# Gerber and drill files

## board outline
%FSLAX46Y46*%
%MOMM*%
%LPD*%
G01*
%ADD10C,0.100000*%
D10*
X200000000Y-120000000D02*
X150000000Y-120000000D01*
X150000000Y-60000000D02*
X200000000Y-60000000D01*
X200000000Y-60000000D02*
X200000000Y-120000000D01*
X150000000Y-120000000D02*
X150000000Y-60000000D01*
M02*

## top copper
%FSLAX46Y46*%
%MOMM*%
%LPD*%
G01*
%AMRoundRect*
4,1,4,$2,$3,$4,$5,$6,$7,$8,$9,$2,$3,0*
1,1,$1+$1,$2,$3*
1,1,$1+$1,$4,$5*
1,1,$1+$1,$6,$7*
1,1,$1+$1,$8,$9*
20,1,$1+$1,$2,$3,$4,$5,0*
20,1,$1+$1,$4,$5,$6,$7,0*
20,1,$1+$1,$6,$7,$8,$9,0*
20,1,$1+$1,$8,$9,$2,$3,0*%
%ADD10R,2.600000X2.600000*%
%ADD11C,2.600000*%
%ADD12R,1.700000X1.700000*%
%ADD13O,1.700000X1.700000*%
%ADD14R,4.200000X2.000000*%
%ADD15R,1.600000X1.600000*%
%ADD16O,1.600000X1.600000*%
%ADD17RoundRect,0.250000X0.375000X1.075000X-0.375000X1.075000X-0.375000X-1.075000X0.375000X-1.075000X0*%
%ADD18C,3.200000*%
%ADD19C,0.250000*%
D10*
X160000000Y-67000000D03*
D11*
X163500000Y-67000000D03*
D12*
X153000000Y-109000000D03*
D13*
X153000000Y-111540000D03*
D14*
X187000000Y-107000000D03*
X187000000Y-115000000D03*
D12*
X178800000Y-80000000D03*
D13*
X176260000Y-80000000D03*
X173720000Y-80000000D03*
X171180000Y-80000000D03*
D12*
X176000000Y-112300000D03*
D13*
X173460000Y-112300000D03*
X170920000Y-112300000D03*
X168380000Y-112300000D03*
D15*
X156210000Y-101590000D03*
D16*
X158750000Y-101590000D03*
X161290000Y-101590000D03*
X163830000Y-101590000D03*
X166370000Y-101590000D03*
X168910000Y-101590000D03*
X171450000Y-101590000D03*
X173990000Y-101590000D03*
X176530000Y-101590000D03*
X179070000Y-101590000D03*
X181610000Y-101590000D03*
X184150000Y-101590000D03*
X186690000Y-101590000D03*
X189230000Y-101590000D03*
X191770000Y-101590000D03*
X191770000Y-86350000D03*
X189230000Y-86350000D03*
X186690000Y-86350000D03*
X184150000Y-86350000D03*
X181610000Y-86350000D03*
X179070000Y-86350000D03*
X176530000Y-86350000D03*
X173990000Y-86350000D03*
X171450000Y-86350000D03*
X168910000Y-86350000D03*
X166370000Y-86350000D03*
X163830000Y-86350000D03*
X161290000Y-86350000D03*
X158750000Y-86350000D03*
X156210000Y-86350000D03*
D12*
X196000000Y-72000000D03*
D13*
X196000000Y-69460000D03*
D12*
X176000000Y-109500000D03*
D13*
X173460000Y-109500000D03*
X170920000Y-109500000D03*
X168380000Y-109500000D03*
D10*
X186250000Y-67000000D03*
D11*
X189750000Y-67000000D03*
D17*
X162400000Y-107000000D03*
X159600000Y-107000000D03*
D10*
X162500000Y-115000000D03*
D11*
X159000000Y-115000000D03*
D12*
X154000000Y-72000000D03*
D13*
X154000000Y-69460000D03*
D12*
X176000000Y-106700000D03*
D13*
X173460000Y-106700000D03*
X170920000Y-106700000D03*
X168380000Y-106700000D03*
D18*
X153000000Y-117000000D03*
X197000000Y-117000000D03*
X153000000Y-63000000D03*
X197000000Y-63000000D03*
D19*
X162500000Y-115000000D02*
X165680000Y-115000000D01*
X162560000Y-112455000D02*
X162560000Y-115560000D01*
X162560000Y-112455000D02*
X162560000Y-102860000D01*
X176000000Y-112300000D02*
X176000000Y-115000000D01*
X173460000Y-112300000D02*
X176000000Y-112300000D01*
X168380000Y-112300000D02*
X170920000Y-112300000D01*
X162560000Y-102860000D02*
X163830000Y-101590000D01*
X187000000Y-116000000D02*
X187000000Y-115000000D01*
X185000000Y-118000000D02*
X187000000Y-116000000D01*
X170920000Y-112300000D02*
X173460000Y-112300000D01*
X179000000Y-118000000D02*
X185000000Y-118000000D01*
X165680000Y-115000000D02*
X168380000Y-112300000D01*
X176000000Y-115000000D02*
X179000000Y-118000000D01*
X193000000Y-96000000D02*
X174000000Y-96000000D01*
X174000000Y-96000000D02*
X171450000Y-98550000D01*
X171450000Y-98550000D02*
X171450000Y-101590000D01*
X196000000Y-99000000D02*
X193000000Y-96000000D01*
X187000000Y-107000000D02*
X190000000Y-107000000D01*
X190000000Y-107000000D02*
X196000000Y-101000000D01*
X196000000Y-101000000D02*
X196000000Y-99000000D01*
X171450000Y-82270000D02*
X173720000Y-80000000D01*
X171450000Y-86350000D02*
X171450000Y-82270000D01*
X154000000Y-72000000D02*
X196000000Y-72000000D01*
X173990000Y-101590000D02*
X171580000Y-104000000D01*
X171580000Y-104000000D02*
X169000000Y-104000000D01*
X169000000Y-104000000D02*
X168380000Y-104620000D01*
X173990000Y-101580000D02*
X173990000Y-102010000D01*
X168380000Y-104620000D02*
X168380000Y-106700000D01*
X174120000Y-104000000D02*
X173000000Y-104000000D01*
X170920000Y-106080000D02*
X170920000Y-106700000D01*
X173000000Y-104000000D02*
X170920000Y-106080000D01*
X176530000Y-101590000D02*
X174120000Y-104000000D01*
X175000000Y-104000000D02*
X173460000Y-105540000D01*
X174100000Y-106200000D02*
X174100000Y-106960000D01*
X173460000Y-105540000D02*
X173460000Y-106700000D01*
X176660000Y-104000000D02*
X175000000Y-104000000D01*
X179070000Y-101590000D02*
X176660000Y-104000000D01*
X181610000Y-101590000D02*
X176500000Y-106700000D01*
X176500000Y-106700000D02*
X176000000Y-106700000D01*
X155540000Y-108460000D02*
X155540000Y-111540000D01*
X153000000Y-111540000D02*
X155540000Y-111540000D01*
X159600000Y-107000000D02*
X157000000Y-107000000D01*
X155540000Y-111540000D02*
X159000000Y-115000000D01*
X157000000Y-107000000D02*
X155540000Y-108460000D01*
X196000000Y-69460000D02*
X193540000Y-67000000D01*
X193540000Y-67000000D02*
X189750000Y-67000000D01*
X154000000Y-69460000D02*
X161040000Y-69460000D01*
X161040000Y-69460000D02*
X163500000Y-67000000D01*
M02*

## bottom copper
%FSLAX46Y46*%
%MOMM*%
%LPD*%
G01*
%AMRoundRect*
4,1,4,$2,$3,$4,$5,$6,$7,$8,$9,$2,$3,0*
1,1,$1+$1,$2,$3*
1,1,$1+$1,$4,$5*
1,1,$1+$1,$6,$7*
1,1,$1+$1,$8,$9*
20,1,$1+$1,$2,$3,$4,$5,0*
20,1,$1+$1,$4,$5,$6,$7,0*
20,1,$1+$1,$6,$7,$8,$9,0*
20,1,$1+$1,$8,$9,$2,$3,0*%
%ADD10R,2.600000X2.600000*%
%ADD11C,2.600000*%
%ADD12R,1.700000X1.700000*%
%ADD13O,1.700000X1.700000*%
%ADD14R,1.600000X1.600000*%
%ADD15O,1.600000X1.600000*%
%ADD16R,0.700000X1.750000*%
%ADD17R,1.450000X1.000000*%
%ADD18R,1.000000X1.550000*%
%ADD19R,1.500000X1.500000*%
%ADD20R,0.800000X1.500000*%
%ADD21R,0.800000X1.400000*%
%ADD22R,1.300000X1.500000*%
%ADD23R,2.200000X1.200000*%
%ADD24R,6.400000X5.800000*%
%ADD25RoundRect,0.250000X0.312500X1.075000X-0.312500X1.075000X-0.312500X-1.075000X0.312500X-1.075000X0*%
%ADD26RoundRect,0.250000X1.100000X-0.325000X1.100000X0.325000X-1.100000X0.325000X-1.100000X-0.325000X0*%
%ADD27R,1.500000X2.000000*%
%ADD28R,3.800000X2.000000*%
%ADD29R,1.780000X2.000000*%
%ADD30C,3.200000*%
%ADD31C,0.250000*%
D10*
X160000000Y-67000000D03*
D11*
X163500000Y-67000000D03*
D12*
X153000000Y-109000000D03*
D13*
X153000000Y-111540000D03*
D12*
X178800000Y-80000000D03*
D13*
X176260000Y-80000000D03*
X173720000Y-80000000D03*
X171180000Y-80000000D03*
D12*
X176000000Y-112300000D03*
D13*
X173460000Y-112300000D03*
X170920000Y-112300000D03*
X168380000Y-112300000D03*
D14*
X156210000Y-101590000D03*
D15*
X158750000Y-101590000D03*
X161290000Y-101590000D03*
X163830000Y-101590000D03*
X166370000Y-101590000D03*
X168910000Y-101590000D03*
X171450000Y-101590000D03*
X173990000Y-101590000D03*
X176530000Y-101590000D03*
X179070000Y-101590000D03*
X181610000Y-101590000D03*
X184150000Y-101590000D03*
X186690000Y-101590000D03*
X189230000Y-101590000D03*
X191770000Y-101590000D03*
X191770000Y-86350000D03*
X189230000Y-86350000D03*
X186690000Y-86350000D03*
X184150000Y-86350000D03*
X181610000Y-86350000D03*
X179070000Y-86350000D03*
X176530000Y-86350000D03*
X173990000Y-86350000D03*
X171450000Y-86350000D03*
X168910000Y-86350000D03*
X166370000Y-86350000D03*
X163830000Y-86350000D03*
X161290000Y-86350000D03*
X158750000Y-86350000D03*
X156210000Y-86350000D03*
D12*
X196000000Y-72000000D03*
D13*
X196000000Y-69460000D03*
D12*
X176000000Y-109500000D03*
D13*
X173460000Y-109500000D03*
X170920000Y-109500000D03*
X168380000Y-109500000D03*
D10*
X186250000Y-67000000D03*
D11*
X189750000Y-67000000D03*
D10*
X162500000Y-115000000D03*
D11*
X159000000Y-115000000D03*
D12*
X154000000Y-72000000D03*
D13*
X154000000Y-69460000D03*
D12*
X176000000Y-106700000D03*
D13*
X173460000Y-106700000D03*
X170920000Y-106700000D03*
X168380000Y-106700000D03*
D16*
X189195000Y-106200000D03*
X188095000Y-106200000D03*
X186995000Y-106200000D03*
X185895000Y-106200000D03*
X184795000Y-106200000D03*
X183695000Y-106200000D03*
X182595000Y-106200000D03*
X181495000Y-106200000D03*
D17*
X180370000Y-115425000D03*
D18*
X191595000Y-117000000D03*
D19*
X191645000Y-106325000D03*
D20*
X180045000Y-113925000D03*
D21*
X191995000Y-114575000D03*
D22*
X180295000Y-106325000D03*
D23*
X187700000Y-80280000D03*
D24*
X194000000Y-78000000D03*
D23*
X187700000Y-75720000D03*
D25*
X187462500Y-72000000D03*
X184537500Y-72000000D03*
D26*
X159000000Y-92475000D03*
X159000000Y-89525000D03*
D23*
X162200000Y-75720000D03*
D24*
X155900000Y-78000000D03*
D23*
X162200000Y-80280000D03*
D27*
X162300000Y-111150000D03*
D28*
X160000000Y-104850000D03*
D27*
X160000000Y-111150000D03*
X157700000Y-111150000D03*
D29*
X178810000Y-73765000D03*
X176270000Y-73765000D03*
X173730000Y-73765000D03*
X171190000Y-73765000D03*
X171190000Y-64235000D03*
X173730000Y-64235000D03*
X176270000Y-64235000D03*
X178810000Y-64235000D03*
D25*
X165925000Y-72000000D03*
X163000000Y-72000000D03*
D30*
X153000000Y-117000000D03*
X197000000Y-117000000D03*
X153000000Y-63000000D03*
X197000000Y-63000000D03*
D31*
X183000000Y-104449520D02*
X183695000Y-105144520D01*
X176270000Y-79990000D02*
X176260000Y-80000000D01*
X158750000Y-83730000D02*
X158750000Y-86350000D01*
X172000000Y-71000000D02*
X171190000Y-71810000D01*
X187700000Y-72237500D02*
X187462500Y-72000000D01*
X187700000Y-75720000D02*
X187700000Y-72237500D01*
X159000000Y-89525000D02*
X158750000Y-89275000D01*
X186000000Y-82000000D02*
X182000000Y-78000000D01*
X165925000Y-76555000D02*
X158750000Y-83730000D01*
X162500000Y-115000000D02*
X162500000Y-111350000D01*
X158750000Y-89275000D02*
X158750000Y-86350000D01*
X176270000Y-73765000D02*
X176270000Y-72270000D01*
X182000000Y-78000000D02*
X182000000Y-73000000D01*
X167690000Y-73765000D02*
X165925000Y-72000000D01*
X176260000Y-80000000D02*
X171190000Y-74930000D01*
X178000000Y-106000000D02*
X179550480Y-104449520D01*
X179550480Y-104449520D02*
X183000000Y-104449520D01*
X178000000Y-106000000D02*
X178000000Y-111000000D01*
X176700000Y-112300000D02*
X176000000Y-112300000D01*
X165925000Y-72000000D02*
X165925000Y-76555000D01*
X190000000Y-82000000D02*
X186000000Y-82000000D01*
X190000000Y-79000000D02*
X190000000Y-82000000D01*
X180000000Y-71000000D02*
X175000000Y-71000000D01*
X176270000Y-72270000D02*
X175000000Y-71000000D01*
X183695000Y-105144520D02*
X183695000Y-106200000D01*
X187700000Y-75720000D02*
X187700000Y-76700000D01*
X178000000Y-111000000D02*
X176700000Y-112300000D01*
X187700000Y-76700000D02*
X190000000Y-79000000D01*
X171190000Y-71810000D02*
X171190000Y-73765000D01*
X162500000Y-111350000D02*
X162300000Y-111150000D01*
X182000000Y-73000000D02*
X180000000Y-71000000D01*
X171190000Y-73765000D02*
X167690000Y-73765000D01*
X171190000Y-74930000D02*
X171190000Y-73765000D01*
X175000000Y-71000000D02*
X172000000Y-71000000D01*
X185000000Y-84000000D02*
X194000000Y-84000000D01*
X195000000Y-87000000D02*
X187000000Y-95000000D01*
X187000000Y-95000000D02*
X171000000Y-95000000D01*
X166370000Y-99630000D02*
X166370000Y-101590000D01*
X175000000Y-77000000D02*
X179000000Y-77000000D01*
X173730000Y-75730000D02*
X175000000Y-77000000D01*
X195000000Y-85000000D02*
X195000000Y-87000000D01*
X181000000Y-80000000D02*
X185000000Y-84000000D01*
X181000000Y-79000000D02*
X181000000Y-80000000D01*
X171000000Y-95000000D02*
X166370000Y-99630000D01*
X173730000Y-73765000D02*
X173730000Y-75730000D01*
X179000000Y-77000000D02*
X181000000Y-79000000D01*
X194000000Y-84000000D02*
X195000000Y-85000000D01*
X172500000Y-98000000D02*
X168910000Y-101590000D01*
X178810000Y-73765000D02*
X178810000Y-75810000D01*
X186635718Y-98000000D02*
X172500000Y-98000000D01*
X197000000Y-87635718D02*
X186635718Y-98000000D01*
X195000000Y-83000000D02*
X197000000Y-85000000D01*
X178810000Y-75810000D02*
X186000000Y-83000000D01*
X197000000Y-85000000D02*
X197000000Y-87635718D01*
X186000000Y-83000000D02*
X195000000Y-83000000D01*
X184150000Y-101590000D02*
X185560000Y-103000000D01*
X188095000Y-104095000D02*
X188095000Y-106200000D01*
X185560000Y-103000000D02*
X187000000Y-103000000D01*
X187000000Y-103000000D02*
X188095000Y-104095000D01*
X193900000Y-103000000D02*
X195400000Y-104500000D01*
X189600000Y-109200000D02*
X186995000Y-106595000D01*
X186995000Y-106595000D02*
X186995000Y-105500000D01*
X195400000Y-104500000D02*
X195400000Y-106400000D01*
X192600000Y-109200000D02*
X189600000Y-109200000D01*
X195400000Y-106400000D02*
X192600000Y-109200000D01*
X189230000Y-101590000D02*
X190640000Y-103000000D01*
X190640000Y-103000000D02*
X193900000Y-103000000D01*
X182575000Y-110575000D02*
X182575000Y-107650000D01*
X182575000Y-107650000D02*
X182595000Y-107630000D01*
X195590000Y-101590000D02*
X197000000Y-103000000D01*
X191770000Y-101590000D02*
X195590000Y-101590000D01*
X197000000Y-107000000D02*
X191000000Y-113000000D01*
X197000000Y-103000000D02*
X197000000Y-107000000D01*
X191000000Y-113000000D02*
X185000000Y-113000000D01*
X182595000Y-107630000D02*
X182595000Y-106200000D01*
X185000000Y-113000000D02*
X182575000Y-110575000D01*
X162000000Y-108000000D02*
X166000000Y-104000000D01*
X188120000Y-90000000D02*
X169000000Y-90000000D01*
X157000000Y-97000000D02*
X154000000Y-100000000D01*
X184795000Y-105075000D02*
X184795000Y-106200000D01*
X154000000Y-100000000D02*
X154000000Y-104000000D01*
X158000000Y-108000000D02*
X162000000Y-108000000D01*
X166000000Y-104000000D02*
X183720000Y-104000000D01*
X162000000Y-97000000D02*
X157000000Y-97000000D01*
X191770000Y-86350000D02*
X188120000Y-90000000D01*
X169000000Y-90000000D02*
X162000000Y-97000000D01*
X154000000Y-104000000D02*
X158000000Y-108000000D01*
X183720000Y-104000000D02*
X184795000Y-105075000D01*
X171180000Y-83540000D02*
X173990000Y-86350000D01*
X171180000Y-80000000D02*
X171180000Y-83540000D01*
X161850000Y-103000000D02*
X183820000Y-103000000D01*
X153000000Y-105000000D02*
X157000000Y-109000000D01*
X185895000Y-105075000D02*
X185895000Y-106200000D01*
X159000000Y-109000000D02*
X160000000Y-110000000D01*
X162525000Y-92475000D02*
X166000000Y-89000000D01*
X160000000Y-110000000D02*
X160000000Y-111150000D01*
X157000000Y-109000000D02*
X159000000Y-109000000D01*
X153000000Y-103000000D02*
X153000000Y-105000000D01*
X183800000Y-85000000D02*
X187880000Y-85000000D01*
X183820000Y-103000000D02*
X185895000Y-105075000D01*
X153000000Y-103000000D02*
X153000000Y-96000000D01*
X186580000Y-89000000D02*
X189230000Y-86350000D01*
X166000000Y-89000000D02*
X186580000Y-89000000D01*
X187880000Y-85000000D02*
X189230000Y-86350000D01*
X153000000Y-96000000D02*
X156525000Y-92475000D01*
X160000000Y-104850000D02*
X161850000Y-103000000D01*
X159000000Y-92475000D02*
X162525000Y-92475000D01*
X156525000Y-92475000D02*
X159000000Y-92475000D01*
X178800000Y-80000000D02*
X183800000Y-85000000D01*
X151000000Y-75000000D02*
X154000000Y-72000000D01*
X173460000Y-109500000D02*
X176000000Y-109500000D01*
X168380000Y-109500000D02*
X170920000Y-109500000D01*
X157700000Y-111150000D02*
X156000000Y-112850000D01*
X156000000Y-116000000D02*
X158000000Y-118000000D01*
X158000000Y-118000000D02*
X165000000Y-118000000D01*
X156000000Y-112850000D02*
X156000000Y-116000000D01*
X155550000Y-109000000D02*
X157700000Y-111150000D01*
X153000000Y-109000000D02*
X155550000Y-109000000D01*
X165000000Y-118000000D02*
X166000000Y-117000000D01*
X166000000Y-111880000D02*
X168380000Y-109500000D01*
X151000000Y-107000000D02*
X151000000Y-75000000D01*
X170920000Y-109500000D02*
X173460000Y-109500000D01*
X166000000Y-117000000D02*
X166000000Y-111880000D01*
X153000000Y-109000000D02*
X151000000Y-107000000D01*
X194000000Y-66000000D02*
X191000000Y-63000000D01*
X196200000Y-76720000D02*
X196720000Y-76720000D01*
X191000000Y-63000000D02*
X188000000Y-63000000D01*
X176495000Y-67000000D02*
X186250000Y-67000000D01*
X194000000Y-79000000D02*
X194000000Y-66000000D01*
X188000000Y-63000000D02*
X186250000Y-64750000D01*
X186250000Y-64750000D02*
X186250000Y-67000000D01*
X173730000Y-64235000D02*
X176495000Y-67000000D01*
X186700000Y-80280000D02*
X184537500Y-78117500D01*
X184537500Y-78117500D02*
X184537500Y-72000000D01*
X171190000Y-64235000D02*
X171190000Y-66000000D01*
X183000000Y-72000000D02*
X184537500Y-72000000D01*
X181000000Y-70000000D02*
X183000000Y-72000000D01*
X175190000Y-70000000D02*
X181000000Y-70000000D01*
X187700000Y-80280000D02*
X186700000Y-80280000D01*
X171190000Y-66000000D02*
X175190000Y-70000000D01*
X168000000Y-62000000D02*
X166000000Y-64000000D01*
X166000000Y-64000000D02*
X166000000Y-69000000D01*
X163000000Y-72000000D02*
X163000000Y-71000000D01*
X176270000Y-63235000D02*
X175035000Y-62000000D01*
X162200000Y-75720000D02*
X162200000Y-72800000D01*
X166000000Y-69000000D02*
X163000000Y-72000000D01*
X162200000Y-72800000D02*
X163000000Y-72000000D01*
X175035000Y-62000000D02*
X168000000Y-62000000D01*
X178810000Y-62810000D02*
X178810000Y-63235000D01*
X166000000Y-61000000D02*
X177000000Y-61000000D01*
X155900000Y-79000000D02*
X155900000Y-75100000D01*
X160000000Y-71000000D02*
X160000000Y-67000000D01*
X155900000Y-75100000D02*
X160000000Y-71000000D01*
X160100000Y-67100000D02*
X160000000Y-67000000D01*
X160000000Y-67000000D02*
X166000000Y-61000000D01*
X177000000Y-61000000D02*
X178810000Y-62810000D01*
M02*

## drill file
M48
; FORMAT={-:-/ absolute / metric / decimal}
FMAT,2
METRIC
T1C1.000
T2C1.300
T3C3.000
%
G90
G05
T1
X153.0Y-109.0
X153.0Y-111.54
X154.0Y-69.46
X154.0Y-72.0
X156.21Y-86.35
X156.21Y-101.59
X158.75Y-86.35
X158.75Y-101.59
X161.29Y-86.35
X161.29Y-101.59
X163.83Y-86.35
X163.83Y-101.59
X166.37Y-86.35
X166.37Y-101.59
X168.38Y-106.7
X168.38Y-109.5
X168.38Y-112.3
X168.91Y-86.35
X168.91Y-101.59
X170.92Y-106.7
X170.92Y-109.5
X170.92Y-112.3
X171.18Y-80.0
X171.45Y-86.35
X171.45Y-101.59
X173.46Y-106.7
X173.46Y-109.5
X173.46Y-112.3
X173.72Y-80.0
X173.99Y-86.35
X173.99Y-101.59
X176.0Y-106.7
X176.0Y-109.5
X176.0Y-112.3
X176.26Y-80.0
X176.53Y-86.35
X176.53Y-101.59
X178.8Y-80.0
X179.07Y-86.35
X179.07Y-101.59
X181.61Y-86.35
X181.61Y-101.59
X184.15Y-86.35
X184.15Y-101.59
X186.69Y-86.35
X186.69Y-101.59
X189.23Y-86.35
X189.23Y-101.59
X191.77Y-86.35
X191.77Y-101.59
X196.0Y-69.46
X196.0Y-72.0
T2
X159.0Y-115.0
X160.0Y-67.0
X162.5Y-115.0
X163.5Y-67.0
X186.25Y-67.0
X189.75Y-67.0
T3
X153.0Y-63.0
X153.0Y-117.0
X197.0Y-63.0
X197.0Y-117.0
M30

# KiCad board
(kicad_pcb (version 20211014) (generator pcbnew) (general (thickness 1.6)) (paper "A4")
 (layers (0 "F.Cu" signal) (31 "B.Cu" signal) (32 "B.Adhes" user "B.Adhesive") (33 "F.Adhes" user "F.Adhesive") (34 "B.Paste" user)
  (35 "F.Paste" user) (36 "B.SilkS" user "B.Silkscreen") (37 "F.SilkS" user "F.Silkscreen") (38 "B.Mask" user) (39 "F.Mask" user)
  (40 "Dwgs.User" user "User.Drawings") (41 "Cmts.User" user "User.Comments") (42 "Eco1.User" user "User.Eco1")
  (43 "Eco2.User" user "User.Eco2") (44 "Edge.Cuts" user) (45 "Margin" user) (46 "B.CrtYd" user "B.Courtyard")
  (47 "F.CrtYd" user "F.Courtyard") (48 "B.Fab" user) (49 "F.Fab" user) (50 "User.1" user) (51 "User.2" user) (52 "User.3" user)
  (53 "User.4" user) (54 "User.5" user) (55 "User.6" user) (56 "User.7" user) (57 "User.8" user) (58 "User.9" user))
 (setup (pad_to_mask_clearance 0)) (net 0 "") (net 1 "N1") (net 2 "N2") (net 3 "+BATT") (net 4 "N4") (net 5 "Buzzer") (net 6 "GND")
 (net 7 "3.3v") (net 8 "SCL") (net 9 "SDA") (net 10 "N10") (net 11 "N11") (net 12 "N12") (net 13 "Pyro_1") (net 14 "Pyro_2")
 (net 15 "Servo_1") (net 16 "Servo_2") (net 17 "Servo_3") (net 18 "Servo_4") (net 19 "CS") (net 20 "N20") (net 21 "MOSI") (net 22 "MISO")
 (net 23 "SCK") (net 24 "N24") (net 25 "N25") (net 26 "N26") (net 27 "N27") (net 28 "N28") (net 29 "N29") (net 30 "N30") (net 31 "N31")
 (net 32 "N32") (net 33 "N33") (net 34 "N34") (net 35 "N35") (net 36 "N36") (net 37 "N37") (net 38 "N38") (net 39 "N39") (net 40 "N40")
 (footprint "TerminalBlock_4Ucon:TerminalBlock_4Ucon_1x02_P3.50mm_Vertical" (layer "F.Cu") (at 160 67)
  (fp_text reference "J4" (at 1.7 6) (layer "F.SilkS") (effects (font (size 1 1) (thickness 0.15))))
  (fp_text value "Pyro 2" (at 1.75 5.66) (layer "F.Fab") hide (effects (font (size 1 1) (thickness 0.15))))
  (pad "1" thru_hole rect (at 0 0) (size 2.6 2.6) (drill 1.3) (layers *.Cu *.Mask) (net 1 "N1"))
  (pad "2" thru_hole circle (at 3.5 0) (size 2.6 2.6) (drill 1.3) (layers *.Cu *.Mask) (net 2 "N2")))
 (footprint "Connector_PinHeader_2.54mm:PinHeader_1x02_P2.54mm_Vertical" (layer "F.Cu") (at 153 109)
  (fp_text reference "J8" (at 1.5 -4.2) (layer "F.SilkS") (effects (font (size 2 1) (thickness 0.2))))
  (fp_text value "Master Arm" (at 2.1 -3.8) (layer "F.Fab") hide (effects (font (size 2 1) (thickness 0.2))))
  (pad "1" thru_hole rect (at 0 0) (size 1.7 1.7) (drill 1) (layers *.Cu *.Mask) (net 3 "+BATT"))
  (pad "2" thru_hole oval (at 0 2.54) (size 1.7 1.7) (drill 1) (layers *.Cu *.Mask) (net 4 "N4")))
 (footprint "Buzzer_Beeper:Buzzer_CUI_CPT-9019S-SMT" (layer "F.Cu") (at 187 111 -90)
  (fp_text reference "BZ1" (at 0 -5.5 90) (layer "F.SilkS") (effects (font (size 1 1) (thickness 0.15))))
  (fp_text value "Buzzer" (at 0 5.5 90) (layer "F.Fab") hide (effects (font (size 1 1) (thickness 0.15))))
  (pad "1" smd rect (at -4 0 270) (size 2 4.2) (layers "F.Cu" "F.Paste" "F.Mask") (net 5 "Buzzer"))
  (pad "2" smd rect (at 4 0 270) (size 2 4.2) (layers "F.Cu" "F.Paste" "F.Mask") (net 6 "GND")))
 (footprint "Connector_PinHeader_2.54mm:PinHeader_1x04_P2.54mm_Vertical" (layer "F.Cu") (at 178.8 80 -90)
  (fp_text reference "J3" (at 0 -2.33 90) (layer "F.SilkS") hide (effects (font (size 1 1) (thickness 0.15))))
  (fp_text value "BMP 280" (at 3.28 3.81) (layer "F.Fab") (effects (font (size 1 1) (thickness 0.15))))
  (pad "1" thru_hole rect (at 0 0 270) (size 1.7 1.7) (drill 1) (layers *.Cu *.Mask) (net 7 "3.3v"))
  (pad "2" thru_hole oval (at 0 2.54 270) (size 1.7 1.7) (drill 1) (layers *.Cu *.Mask) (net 6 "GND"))
  (pad "3" thru_hole oval (at 0 5.08 270) (size 1.7 1.7) (drill 1) (layers *.Cu *.Mask) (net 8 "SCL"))
  (pad "4" thru_hole oval (at 0 7.62 270) (size 1.7 1.7) (drill 1) (layers *.Cu *.Mask) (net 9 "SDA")))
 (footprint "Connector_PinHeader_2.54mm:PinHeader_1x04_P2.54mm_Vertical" (layer "F.Cu") (at 176 112.3 -90)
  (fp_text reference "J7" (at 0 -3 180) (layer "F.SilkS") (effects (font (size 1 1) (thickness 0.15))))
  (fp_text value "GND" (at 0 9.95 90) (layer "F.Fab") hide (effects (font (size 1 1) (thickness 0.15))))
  (pad "1" thru_hole rect (at 0 0 270) (size 1.7 1.7) (drill 1) (layers *.Cu *.Mask) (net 6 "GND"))
  (pad "2" thru_hole oval (at 0 2.54 270) (size 1.7 1.7) (drill 1) (layers *.Cu *.Mask) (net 6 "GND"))
  (pad "3" thru_hole oval (at 0 5.08 270) (size 1.7 1.7) (drill 1) (layers *.Cu *.Mask) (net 6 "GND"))
  (pad "4" thru_hole oval (at 0 7.62 270) (size 1.7 1.7) (drill 1) (layers *.Cu *.Mask) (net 6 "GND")))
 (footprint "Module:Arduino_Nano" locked (layer "F.Cu") (at 156.21 101.59 90)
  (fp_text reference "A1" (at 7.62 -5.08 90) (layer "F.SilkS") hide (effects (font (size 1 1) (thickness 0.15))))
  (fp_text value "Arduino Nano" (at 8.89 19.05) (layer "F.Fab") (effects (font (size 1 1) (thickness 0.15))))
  (pad "1" thru_hole rect locked (at 0 0 90) (size 1.6 1.6) (drill 1) (layers *.Cu *.Mask) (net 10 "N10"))
  (pad "2" thru_hole oval locked (at 0 2.54 90) (size 1.6 1.6) (drill 1) (layers *.Cu *.Mask) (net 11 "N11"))
  (pad "3" thru_hole oval locked (at 0 5.08 90) (size 1.6 1.6) (drill 1) (layers *.Cu *.Mask) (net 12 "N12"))
  (pad "4" thru_hole oval locked (at 0 7.62 90) (size 1.6 1.6) (drill 1) (layers *.Cu *.Mask) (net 6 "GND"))
  (pad "5" thru_hole oval locked (at 0 10.16 90) (size 1.6 1.6) (drill 1) (layers *.Cu *.Mask) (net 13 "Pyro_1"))
  (pad "6" thru_hole oval locked (at 0 12.7 90) (size 1.6 1.6) (drill 1) (layers *.Cu *.Mask) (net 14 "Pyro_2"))
  (pad "7" thru_hole oval locked (at 0 15.24 90) (size 1.6 1.6) (drill 1) (layers *.Cu *.Mask) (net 5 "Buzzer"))
  (pad "8" thru_hole oval locked (at 0 17.78 90) (size 1.6 1.6) (drill 1) (layers *.Cu *.Mask) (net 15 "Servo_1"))
  (pad "9" thru_hole oval locked (at 0 20.32 90) (size 1.6 1.6) (drill 1) (layers *.Cu *.Mask) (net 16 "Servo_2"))
  (pad "10" thru_hole oval locked (at 0 22.86 90) (size 1.6 1.6) (drill 1) (layers *.Cu *.Mask) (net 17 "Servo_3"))
  (pad "11" thru_hole oval locked (at 0 25.4 90) (size 1.6 1.6) (drill 1) (layers *.Cu *.Mask) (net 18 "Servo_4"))
  (pad "12" thru_hole oval locked (at 0 27.94 90) (size 1.6 1.6) (drill 1) (layers *.Cu *.Mask) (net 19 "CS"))
  (pad "13" thru_hole oval locked (at 0 30.48 90) (size 1.6 1.6) (drill 1) (layers *.Cu *.Mask) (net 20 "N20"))
  (pad "14" thru_hole oval locked (at 0 33.02 90) (size 1.6 1.6) (drill 1) (layers *.Cu *.Mask) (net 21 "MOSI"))
  (pad "15" thru_hole oval locked (at 0 35.56 90) (size 1.6 1.6) (drill 1) (layers *.Cu *.Mask) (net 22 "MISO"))
  (pad "16" thru_hole oval locked (at 15.24 35.56 90) (size 1.6 1.6) (drill 1) (layers *.Cu *.Mask) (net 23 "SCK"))
  (pad "17" thru_hole oval locked (at 15.24 33.02 90) (size 1.6 1.6) (drill 1) (layers *.Cu *.Mask) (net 7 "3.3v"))
  (pad "18" thru_hole oval locked (at 15.24 30.48 90) (size 1.6 1.6) (drill 1) (layers *.Cu *.Mask) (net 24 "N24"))
  (pad "19" thru_hole oval locked (at 15.24 27.94 90) (size 1.6 1.6) (drill 1) (layers *.Cu *.Mask) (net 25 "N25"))
  (pad "20" thru_hole oval locked (at 15.24 25.4 90) (size 1.6 1.6) (drill 1) (layers *.Cu *.Mask) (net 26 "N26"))
  (pad "21" thru_hole oval locked (at 15.24 22.86 90) (size 1.6 1.6) (drill 1) (layers *.Cu *.Mask) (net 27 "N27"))
  (pad "22" thru_hole oval locked (at 15.24 20.32 90) (size 1.6 1.6) (drill 1) (layers *.Cu *.Mask) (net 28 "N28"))
  (pad "23" thru_hole oval locked (at 15.24 17.78 90) (size 1.6 1.6) (drill 1) (layers *.Cu *.Mask) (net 9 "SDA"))
  (pad "24" thru_hole oval locked (at 15.24 15.24 90) (size 1.6 1.6) (drill 1) (layers *.Cu *.Mask) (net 8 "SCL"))
  (pad "25" thru_hole oval locked (at 15.24 12.7 90) (size 1.6 1.6) (drill 1) (layers *.Cu *.Mask) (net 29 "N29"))
  (pad "26" thru_hole oval locked (at 15.24 10.16 90) (size 1.6 1.6) (drill 1) (layers *.Cu *.Mask) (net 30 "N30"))
  (pad "27" thru_hole oval locked (at 15.24 7.62 90) (size 1.6 1.6) (drill 1) (layers *.Cu *.Mask) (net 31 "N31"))
  (pad "28" thru_hole oval locked (at 15.24 5.08 90) (size 1.6 1.6) (drill 1) (layers *.Cu *.Mask) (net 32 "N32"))
  (pad "29" thru_hole oval locked (at 15.24 2.54 90) (size 1.6 1.6) (drill 1) (layers *.Cu *.Mask) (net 6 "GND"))
  (pad "30" thru_hole oval locked (at 15.24 0 90) (size 1.6 1.6) (drill 1) (layers *.Cu *.Mask) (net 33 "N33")))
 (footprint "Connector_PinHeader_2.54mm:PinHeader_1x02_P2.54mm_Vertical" (layer "F.Cu") (at 196 72 180)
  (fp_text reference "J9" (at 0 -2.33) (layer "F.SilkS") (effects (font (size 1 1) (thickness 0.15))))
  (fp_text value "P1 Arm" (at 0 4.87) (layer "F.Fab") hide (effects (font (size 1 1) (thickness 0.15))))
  (pad "1" thru_hole rect (at 0 0 180) (size 1.7 1.7) (drill 1) (layers *.Cu *.Mask) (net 3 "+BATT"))
  (pad "2" thru_hole oval (at 0 2.54 180) (size 1.7 1.7) (drill 1) (layers *.Cu *.Mask) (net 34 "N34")))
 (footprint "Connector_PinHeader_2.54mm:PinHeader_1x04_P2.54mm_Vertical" (layer "F.Cu") (at 176 109.5 -90)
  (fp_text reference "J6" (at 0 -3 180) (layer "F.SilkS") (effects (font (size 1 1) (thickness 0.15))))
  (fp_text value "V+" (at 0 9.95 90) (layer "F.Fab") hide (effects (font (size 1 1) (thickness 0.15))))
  (pad "1" thru_hole rect (at 0 0 270) (size 1.7 1.7) (drill 1) (layers *.Cu *.Mask) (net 3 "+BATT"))
  (pad "2" thru_hole oval (at 0 2.54 270) (size 1.7 1.7) (drill 1) (layers *.Cu *.Mask) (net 3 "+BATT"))
  (pad "3" thru_hole oval (at 0 5.08 270) (size 1.7 1.7) (drill 1) (layers *.Cu *.Mask) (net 3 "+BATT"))
  (pad "4" thru_hole oval (at 0 7.62 270) (size 1.7 1.7) (drill 1) (layers *.Cu *.Mask) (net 3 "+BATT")))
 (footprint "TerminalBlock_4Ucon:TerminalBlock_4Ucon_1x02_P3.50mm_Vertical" (layer "F.Cu") (at 186.25 67)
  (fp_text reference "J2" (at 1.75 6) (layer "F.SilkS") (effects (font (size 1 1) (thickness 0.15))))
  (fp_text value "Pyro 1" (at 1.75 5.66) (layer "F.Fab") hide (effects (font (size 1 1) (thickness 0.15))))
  (pad "1" thru_hole rect (at 0 0) (size 2.6 2.6) (drill 1.3) (layers *.Cu *.Mask) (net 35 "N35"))
  (pad "2" thru_hole circle (at 3.5 0) (size 2.6 2.6) (drill 1.3) (layers *.Cu *.Mask) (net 34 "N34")))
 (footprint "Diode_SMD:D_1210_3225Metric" (layer "F.Cu") (at 161 107 180)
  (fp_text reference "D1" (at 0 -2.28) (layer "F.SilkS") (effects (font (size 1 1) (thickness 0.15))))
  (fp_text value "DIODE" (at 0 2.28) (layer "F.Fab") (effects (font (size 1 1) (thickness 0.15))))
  (pad "1" smd roundrect (at -1.4 0 180) (size 1.25 2.65) (layers "F.Cu" "F.Paste" "F.Mask") (roundrect_rratio 0.2) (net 6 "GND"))
  (pad "2" smd roundrect (at 1.4 0 180) (size 1.25 2.65) (layers "F.Cu" "F.Paste" "F.Mask") (roundrect_rratio 0.2) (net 4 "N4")))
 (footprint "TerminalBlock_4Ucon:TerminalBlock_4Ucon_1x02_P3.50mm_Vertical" (layer "F.Cu") (at 162.5 115 180)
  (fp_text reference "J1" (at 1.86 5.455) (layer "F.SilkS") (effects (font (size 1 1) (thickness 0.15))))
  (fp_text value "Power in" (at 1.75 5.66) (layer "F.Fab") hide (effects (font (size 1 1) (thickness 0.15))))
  (pad "1" thru_hole rect (at 0 0 180) (size 2.6 2.6) (drill 1.3) (layers *.Cu *.Mask) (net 6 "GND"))
  (pad "2" thru_hole circle (at 3.5 0 180) (size 2.6 2.6) (drill 1.3) (layers *.Cu *.Mask) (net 4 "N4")))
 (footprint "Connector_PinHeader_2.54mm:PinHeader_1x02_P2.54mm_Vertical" (layer "F.Cu") (at 154 72 180)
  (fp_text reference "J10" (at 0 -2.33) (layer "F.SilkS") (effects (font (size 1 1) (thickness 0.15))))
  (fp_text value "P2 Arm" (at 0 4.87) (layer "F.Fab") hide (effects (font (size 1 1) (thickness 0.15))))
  (pad "1" thru_hole rect (at 0 0 180) (size 1.7 1.7) (drill 1) (layers *.Cu *.Mask) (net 3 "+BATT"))
  (pad "2" thru_hole oval (at 0 2.54 180) (size 1.7 1.7) (drill 1) (layers *.Cu *.Mask) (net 2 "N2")))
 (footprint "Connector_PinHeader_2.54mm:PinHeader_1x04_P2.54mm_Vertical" (layer "F.Cu") (at 176 106.7 -90)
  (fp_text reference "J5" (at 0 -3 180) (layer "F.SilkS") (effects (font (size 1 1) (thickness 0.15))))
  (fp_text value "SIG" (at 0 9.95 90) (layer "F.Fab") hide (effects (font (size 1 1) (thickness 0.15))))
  (pad "1" thru_hole rect (at 0 0 270) (size 1.7 1.7) (drill 1) (layers *.Cu *.Mask) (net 18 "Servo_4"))
  (pad "2" thru_hole oval (at 0 2.54 270) (size 1.7 1.7) (drill 1) (layers *.Cu *.Mask) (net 17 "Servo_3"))
  (pad "3" thru_hole oval (at 0 5.08 270) (size 1.7 1.7) (drill 1) (layers *.Cu *.Mask) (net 16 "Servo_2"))
  (pad "4" thru_hole oval (at 0 7.62 270) (size 1.7 1.7) (drill 1) (layers *.Cu *.Mask) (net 15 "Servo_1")))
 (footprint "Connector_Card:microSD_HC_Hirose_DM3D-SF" (layer "B.Cu") (at 186.02 111.55)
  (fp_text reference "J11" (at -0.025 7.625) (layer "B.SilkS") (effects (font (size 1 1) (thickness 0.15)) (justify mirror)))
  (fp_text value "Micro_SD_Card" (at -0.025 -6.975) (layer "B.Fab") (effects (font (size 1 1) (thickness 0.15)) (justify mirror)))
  (pad "1" smd rect locked (at 3.175 -5.35) (size 0.7 1.75) (layers "B.Cu" "B.Paste" "B.Mask") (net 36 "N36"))
  (pad "2" smd rect locked (at 2.075 -5.35) (size 0.7 1.75) (layers "B.Cu" "B.Paste" "B.Mask") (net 19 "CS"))
  (pad "3" smd rect locked (at 0.975 -5.35) (size 0.7 1.75) (layers "B.Cu" "B.Paste" "B.Mask") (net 21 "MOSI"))
  (pad "4" smd rect locked (at -0.125 -5.35) (size 0.7 1.75) (layers "B.Cu" "B.Paste" "B.Mask") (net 7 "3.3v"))
  (pad "5" smd rect locked (at -1.225 -5.35) (size 0.7 1.75) (layers "B.Cu" "B.Paste" "B.Mask") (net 23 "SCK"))
  (pad "6" smd rect locked (at -2.325 -5.35) (size 0.7 1.75) (layers "B.Cu" "B.Paste" "B.Mask") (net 6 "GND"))
  (pad "7" smd rect locked (at -3.425 -5.35) (size 0.7 1.75) (layers "B.Cu" "B.Paste" "B.Mask") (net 22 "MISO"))
  (pad "8" smd rect locked (at -4.525 -5.35) (size 0.7 1.75) (layers "B.Cu" "B.Paste" "B.Mask") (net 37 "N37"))
  (pad "9" smd rect locked (at -5.65 3.875) (size 1.45 1) (layers "B.Cu" "B.Paste" "B.Mask") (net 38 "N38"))
  (pad "10" smd rect locked (at 5.575 5.45) (size 1 1.55) (layers "B.Cu" "B.Paste" "B.Mask"))
  (pad "11" smd rect locked (at 5.625 -5.225) (size 1.5 1.5) (layers "B.Cu" "B.Paste" "B.Mask"))
  (pad "11" smd rect locked (at -5.975 2.375) (size 0.8 1.5) (layers "B.Cu" "B.Paste" "B.Mask"))
  (pad "11" smd rect locked (at 5.975 3.025) (size 0.8 1.4) (layers "B.Cu" "B.Paste" "B.Mask"))
  (pad "11" smd rect locked (at -5.725 -5.225) (size 1.3 1.5) (layers "B.Cu" "B.Paste" "B.Mask")))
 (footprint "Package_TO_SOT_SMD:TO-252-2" (layer "B.Cu") (at 191.9 78)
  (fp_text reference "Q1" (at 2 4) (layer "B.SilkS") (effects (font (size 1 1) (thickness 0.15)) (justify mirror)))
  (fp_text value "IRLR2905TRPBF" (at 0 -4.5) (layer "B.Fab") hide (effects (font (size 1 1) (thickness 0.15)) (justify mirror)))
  (pad "" smd rect (at 0.425 1.525) (size 3.05 2.75) (layers "B.Paste"))
  (pad "" smd rect (at 0.425 -1.525) (size 3.05 2.75) (layers "B.Paste"))
  (pad "" smd rect (at 3.775 1.525) (size 3.05 2.75) (layers "B.Paste"))
  (pad "" smd rect (at 3.775 -1.525) (size 3.05 2.75) (layers "B.Paste"))
  (pad "1" smd rect (at -4.2 2.28) (size 2.2 1.2) (layers "B.Cu" "B.Paste" "B.Mask") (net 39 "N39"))
  (pad "2" smd rect (at 2.1 0) (size 6.4 5.8) (layers "B.Cu" "B.Mask") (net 35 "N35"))
  (pad "3" smd rect (at -4.2 -2.28) (size 2.2 1.2) (layers "B.Cu" "B.Paste" "B.Mask") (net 6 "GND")))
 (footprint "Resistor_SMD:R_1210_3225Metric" (layer "B.Cu") (at 186 72 180)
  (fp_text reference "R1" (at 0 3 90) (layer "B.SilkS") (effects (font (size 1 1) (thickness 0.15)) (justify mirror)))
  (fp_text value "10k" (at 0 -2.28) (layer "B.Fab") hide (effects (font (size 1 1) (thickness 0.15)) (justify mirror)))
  (pad "1" smd roundrect (at -1.4625 0 180) (size 1.125 2.65) (layers "B.Cu" "B.Paste" "B.Mask") (roundrect_rratio 0.2222222222)
   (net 6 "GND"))
  (pad "2" smd roundrect (at 1.4625 0 180) (size 1.125 2.65) (layers "B.Cu" "B.Paste" "B.Mask") (roundrect_rratio 0.2222222222)
   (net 39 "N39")))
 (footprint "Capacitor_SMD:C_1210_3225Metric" (layer "B.Cu") (at 159 91 90)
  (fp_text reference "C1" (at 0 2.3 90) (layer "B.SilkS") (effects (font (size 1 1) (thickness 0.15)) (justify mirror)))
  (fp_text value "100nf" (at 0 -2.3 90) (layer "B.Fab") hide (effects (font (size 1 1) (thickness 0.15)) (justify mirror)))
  (pad "1" smd roundrect (at -1.475 0 90) (size 1.15 2.7) (layers "B.Cu" "B.Paste" "B.Mask") (roundrect_rratio 0.2173913043) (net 7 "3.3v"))
  (pad "2" smd roundrect (at 1.475 0 90) (size 1.15 2.7) (layers "B.Cu" "B.Paste" "B.Mask") (roundrect_rratio 0.2173913043) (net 6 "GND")))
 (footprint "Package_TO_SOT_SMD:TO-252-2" (layer "B.Cu") (at 158 78 180)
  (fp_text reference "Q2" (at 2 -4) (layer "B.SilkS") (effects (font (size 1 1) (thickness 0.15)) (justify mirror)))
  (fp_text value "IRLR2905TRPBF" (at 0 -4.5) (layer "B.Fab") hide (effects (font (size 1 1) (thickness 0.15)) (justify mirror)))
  (pad "" smd rect (at 0.425 -1.525 180) (size 3.05 2.75) (layers "B.Paste"))
  (pad "" smd rect (at 3.775 -1.525 180) (size 3.05 2.75) (layers "B.Paste"))
  (pad "" smd rect (at 3.775 1.525 180) (size 3.05 2.75) (layers "B.Paste"))
  (pad "" smd rect (at 0.425 1.525 180) (size 3.05 2.75) (layers "B.Paste"))
  (pad "1" smd rect (at -4.2 2.28 180) (size 2.2 1.2) (layers "B.Cu" "B.Paste" "B.Mask") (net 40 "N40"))
  (pad "2" smd rect (at 2.1 0 180) (size 6.4 5.8) (layers "B.Cu" "B.Mask") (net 1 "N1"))
  (pad "3" smd rect (at -4.2 -2.28 180) (size 2.2 1.2) (layers "B.Cu" "B.Paste" "B.Mask") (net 6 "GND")))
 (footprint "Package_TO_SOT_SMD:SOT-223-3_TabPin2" (layer "B.Cu") (at 160 108 90)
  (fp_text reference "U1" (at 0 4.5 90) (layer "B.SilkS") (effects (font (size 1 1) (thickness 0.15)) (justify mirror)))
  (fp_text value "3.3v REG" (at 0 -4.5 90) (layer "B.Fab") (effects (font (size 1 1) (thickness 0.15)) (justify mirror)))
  (pad "1" smd rect (at -3.15 2.3 90) (size 2 1.5) (layers "B.Cu" "B.Paste" "B.Mask") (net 6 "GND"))
  (pad "2" smd rect (at 3.15 0 90) (size 2 3.8) (layers "B.Cu" "B.Paste" "B.Mask") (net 7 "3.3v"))
  (pad "2" smd rect (at -3.15 0 90) (size 2 1.5) (layers "B.Cu" "B.Paste" "B.Mask") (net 7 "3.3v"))
  (pad "3" smd rect (at -3.15 -2.3 90) (size 2 1.5) (layers "B.Cu" "B.Paste" "B.Mask") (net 3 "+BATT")))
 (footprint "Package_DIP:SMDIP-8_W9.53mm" (layer "B.Cu") (at 175 69 90)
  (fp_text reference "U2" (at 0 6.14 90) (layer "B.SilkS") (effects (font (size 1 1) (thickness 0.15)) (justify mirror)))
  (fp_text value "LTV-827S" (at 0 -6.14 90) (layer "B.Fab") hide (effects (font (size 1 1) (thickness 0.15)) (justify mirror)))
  (pad "1" smd rect (at -4.765 3.81 90) (size 2 1.78) (layers "B.Cu" "B.Paste" "B.Mask") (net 14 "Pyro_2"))
  (pad "2" smd rect (at -4.765 1.27 90) (size 2 1.78) (layers "B.Cu" "B.Paste" "B.Mask") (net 6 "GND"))
  (pad "3" smd rect (at -4.765 -1.27 90) (size 2 1.78) (layers "B.Cu" "B.Paste" "B.Mask") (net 13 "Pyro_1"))
  (pad "4" smd rect (at -4.765 -3.81 90) (size 2 1.78) (layers "B.Cu" "B.Paste" "B.Mask") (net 6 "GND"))
  (pad "5" smd rect (at 4.765 -3.81 90) (size 2 1.78) (layers "B.Cu" "B.Paste" "B.Mask") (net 39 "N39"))
  (pad "6" smd rect (at 4.765 -1.27 90) (size 2 1.78) (layers "B.Cu" "B.Paste" "B.Mask") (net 35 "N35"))
  (pad "7" smd rect (at 4.765 1.27 90) (size 2 1.78) (layers "B.Cu" "B.Paste" "B.Mask") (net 40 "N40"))
  (pad "8" smd rect (at 4.765 3.81 90) (size 2 1.78) (layers "B.Cu" "B.Paste" "B.Mask") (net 1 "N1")))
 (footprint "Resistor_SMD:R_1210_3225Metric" (layer "B.Cu") (at 164.4625 72 180)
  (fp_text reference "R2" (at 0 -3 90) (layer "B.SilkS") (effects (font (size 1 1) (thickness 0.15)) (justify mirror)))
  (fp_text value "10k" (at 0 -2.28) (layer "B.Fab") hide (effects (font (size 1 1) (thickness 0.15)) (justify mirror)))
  (pad "1" smd roundrect (at -1.4625 0 180) (size 1.125 2.65) (layers "B.Cu" "B.Paste" "B.Mask") (roundrect_rratio 0.2222222222)
   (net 6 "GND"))
  (pad "2" smd roundrect (at 1.4625 0 180) (size 1.125 2.65) (layers "B.Cu" "B.Paste" "B.Mask") (roundrect_rratio 0.2222222222)
   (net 40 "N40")))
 (gr_line (start 200 120) (end 150 120) (layer "Edge.Cuts") (width 0.1))
 (gr_line (start 150 60) (end 200 60) (layer "Edge.Cuts") (width 0.1))
 (gr_line (start 200 60) (end 200 120) (layer "Edge.Cuts") (width 0.1))
 (gr_line (start 150 120) (end 150 60) (layer "Edge.Cuts") (width 0.1))
 (via (at 153 117) (size 3.2) (drill 3) (layers "F.Cu" "B.Cu") (free) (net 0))
 (via (at 197 117) (size 3.2) (drill 3) (layers "F.Cu" "B.Cu") (free) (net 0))
 (via (at 153 63) (size 3.2) (drill 3) (layers "F.Cu" "B.Cu") (free) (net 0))
 (via (at 197 63) (size 3.2) (drill 3) (layers "F.Cu" "B.Cu") (free) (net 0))
 (segment (start 162.5 115) (end 165.68 115) (width 0.25) (layer "F.Cu") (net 6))
 (segment (start 162.56 112.455) (end 162.56 115.56) (width 0.25) (layer "F.Cu") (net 6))
 (segment (start 162.56 112.455) (end 162.56 102.86) (width 0.25) (layer "F.Cu") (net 6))
 (segment (start 176 112.3) (end 176 115) (width 0.25) (layer "F.Cu") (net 6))
 (segment (start 173.46 112.3) (end 176 112.3) (width 0.25) (layer "F.Cu") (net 6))
 (segment (start 168.38 112.3) (end 170.92 112.3) (width 0.25) (layer "F.Cu") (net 6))
 (segment (start 162.56 102.86) (end 163.83 101.59) (width 0.25) (layer "F.Cu") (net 6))
 (segment (start 187 116) (end 187 115) (width 0.25) (layer "F.Cu") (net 6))
 (segment (start 185 118) (end 187 116) (width 0.25) (layer "F.Cu") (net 6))
 (segment (start 170.92 112.3) (end 173.46 112.3) (width 0.25) (layer "F.Cu") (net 6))
 (segment (start 179 118) (end 185 118) (width 0.25) (layer "F.Cu") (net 6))
 (segment (start 165.68 115) (end 168.38 112.3) (width 0.25) (layer "F.Cu") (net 6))
 (segment (start 176 115) (end 179 118) (width 0.25) (layer "F.Cu") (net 6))
 (segment (start 183 104.44952) (end 183.695 105.14452) (width 0.25) (layer "B.Cu") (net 6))
 (segment (start 176.27 79.99) (end 176.26 80) (width 0.25) (layer "B.Cu") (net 6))
 (segment (start 158.75 83.73) (end 158.75 86.35) (width 0.25) (layer "B.Cu") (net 6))
 (segment (start 172 71) (end 171.19 71.81) (width 0.25) (layer "B.Cu") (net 6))
 (segment (start 187.7 72.2375) (end 187.4625 72) (width 0.25) (layer "B.Cu") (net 6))
 (segment (start 187.7 75.72) (end 187.7 72.2375) (width 0.25) (layer "B.Cu") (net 6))
 (segment (start 159 89.525) (end 158.75 89.275) (width 0.25) (layer "B.Cu") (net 6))
 (segment (start 186 82) (end 182 78) (width 0.25) (layer "B.Cu") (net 6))
 (segment (start 165.925 76.555) (end 158.75 83.73) (width 0.25) (layer "B.Cu") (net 6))
 (segment (start 162.5 115) (end 162.5 111.35) (width 0.25) (layer "B.Cu") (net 6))
 (segment (start 158.75 89.275) (end 158.75 86.35) (width 0.25) (layer "B.Cu") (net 6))
 (segment (start 176.27 73.765) (end 176.27 72.27) (width 0.25) (layer "B.Cu") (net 6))
 (segment (start 182 78) (end 182 73) (width 0.25) (layer "B.Cu") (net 6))
 (segment (start 167.69 73.765) (end 165.925 72) (width 0.25) (layer "B.Cu") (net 6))
 (segment (start 176.26 80) (end 171.19 74.93) (width 0.25) (layer "B.Cu") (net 6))
 (segment (start 178 106) (end 179.55048 104.44952) (width 0.25) (layer "B.Cu") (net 6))
 (segment (start 179.55048 104.44952) (end 183 104.44952) (width 0.25) (layer "B.Cu") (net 6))
 (segment (start 178 106) (end 178 111) (width 0.25) (layer "B.Cu") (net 6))
 (segment (start 176.7 112.3) (end 176 112.3) (width 0.25) (layer "B.Cu") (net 6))
 (segment (start 165.925 72) (end 165.925 76.555) (width 0.25) (layer "B.Cu") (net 6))
 (segment (start 190 82) (end 186 82) (width 0.25) (layer "B.Cu") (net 6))
 (segment (start 190 79) (end 190 82) (width 0.25) (layer "B.Cu") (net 6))
 (segment (start 180 71) (end 175 71) (width 0.25) (layer "B.Cu") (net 6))
 (segment (start 176.27 72.27) (end 175 71) (width 0.25) (layer "B.Cu") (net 6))
 (segment (start 183.695 105.14452) (end 183.695 106.2) (width 0.25) (layer "B.Cu") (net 6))
 (segment (start 187.7 75.72) (end 187.7 76.7) (width 0.25) (layer "B.Cu") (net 6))
 (segment (start 178 111) (end 176.7 112.3) (width 0.25) (layer "B.Cu") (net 6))
 (segment (start 187.7 76.7) (end 190 79) (width 0.25) (layer "B.Cu") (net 6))
 (segment (start 171.19 71.81) (end 171.19 73.765) (width 0.25) (layer "B.Cu") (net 6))
 (segment (start 162.5 111.35) (end 162.3 111.15) (width 0.25) (layer "B.Cu") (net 6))
 (segment (start 182 73) (end 180 71) (width 0.25) (layer "B.Cu") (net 6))
 (segment (start 171.19 73.765) (end 167.69 73.765) (width 0.25) (layer "B.Cu") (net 6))
 (segment (start 171.19 74.93) (end 171.19 73.765) (width 0.25) (layer "B.Cu") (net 6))
 (segment (start 175 71) (end 172 71) (width 0.25) (layer "B.Cu") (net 6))
 (segment (start 185 84) (end 194 84) (width 0.25) (layer "B.Cu") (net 13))
 (segment (start 195 87) (end 187 95) (width 0.25) (layer "B.Cu") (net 13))
 (segment (start 187 95) (end 171 95) (width 0.25) (layer "B.Cu") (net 13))
 (segment (start 166.37 99.63) (end 166.37 101.59) (width 0.25) (layer "B.Cu") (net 13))
 (segment (start 175 77) (end 179 77) (width 0.25) (layer "B.Cu") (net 13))
 (segment (start 173.73 75.73) (end 175 77) (width 0.25) (layer "B.Cu") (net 13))
 (segment (start 195 85) (end 195 87) (width 0.25) (layer "B.Cu") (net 13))
 (segment (start 181 80) (end 185 84) (width 0.25) (layer "B.Cu") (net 13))
 (segment (start 181 79) (end 181 80) (width 0.25) (layer "B.Cu") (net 13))
 (segment (start 171 95) (end 166.37 99.63) (width 0.25) (layer "B.Cu") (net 13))
 (segment (start 173.73 73.765) (end 173.73 75.73) (width 0.25) (layer "B.Cu") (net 13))
 (segment (start 179 77) (end 181 79) (width 0.25) (layer "B.Cu") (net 13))
 (segment (start 194 84) (end 195 85) (width 0.25) (layer "B.Cu") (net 13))
 (segment (start 172.5 98) (end 168.91 101.59) (width 0.25) (layer "B.Cu") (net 14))
 (segment (start 178.81 73.765) (end 178.81 75.81) (width 0.25) (layer "B.Cu") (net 14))
 (segment (start 186.635718 98) (end 172.5 98) (width 0.25) (layer "B.Cu") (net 14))
 (segment (start 197 87.635718) (end 186.635718 98) (width 0.25) (layer "B.Cu") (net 14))
 (segment (start 195 83) (end 197 85) (width 0.25) (layer "B.Cu") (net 14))
 (segment (start 178.81 75.81) (end 186 83) (width 0.25) (layer "B.Cu") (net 14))
 (segment (start 197 85) (end 197 87.635718) (width 0.25) (layer "B.Cu") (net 14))
 (segment (start 186 83) (end 195 83) (width 0.25) (layer "B.Cu") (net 14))
 (segment (start 193 96) (end 174 96) (width 0.25) (layer "F.Cu") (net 5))
 (segment (start 174 96) (end 171.45 98.55) (width 0.25) (layer "F.Cu") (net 5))
 (segment (start 171.45 98.55) (end 171.45 101.59) (width 0.25) (layer "F.Cu") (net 5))
 (segment (start 196 99) (end 193 96) (width 0.25) (layer "F.Cu") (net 5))
 (segment (start 187 107) (end 190 107) (width 0.25) (layer "F.Cu") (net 5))
 (segment (start 190 107) (end 196 101) (width 0.25) (layer "F.Cu") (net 5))
 (segment (start 196 101) (end 196 99) (width 0.25) (layer "F.Cu") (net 5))
 (segment (start 184.15 101.59) (end 185.56 103) (width 0.25) (layer "B.Cu") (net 19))
 (segment (start 188.095 104.095) (end 188.095 106.2) (width 0.25) (layer "B.Cu") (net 19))
 (segment (start 185.56 103) (end 187 103) (width 0.25) (layer "B.Cu") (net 19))
 (segment (start 187 103) (end 188.095 104.095) (width 0.25) (layer "B.Cu") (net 19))
 (segment (start 193.9 103) (end 195.4 104.5) (width 0.25) (layer "B.Cu") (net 21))
 (segment (start 189.6 109.2) (end 186.995 106.595) (width 0.25) (layer "B.Cu") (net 21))
 (segment (start 186.995 106.595) (end 186.995 105.5) (width 0.25) (layer "B.Cu") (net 21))
 (segment (start 195.4 104.5) (end 195.4 106.4) (width 0.25) (layer "B.Cu") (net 21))
 (segment (start 192.6 109.2) (end 189.6 109.2) (width 0.25) (layer "B.Cu") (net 21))
 (segment (start 195.4 106.4) (end 192.6 109.2) (width 0.25) (layer "B.Cu") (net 21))
 (segment (start 189.23 101.59) (end 190.64 103) (width 0.25) (layer "B.Cu") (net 21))
 (segment (start 190.64 103) (end 193.9 103) (width 0.25) (layer "B.Cu") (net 21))
 (segment (start 182.575 110.575) (end 182.575 107.65) (width 0.25) (layer "B.Cu") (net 22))
 (segment (start 182.575 107.65) (end 182.595 107.63) (width 0.25) (layer "B.Cu") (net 22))
 (segment (start 195.59 101.59) (end 197 103) (width 0.25) (layer "B.Cu") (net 22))
 (segment (start 191.77 101.59) (end 195.59 101.59) (width 0.25) (layer "B.Cu") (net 22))
 (segment (start 197 107) (end 191 113) (width 0.25) (layer "B.Cu") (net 22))
 (segment (start 197 103) (end 197 107) (width 0.25) (layer "B.Cu") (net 22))
 (segment (start 191 113) (end 185 113) (width 0.25) (layer "B.Cu") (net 22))
 (segment (start 182.595 107.63) (end 182.595 106.2) (width 0.25) (layer "B.Cu") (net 22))
 (segment (start 185 113) (end 182.575 110.575) (width 0.25) (layer "B.Cu") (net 22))
 (segment (start 162 108) (end 166 104) (width 0.25) (layer "B.Cu") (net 23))
 (segment (start 188.12 90) (end 169 90) (width 0.25) (layer "B.Cu") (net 23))
 (segment (start 157 97) (end 154 100) (width 0.25) (layer "B.Cu") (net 23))
 (segment (start 184.795 105.075) (end 184.795 106.2) (width 0.25) (layer "B.Cu") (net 23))
 (segment (start 154 100) (end 154 104) (width 0.25) (layer "B.Cu") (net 23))
 (segment (start 158 108) (end 162 108) (width 0.25) (layer "B.Cu") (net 23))
 (segment (start 166 104) (end 183.72 104) (width 0.25) (layer "B.Cu") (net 23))
 (segment (start 162 97) (end 157 97) (width 0.25) (layer "B.Cu") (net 23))
 (segment (start 191.77 86.35) (end 188.12 90) (width 0.25) (layer "B.Cu") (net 23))
 (segment (start 169 90) (end 162 97) (width 0.25) (layer "B.Cu") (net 23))
 (segment (start 154 104) (end 158 108) (width 0.25) (layer "B.Cu") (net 23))
 (segment (start 183.72 104) (end 184.795 105.075) (width 0.25) (layer "B.Cu") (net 23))
 (segment (start 171.18 83.54) (end 173.99 86.35) (width 0.25) (layer "B.Cu") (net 9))
 (segment (start 171.18 80) (end 171.18 83.54) (width 0.25) (layer "B.Cu") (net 9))
 (segment (start 171.45 82.27) (end 173.72 80) (width 0.25) (layer "F.Cu") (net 8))
 (segment (start 171.45 86.35) (end 171.45 82.27) (width 0.25) (layer "F.Cu") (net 8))
 (segment (start 161.85 103) (end 183.82 103) (width 0.25) (layer "B.Cu") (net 7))
 (segment (start 153 105) (end 157 109) (width 0.25) (layer "B.Cu") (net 7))
 (segment (start 185.895 105.075) (end 185.895 106.2) (width 0.25) (layer "B.Cu") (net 7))
 (segment (start 159 109) (end 160 110) (width 0.25) (layer "B.Cu") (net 7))
 (segment (start 162.525 92.475) (end 166 89) (width 0.25) (layer "B.Cu") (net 7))
 (segment (start 160 110) (end 160 111.15) (width 0.25) (layer "B.Cu") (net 7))
 (segment (start 157 109) (end 159 109) (width 0.25) (layer "B.Cu") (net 7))
 (segment (start 153 103) (end 153 105) (width 0.25) (layer "B.Cu") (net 7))
 (segment (start 183.8 85) (end 187.88 85) (width 0.25) (layer "B.Cu") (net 7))
 (segment (start 183.82 103) (end 185.895 105.075) (width 0.25) (layer "B.Cu") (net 7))
 (segment (start 153 103) (end 153 96) (width 0.25) (layer "B.Cu") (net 7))
 (segment (start 186.58 89) (end 189.23 86.35) (width 0.25) (layer "B.Cu") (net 7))
 (segment (start 166 89) (end 186.58 89) (width 0.25) (layer "B.Cu") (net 7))
 (segment (start 187.88 85) (end 189.23 86.35) (width 0.25) (layer "B.Cu") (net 7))
 (segment (start 153 96) (end 156.525 92.475) (width 0.25) (layer "B.Cu") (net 7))
 (segment (start 160 104.85) (end 161.85 103) (width 0.25) (layer "B.Cu") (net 7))
 (segment (start 159 92.475) (end 162.525 92.475) (width 0.25) (layer "B.Cu") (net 7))
 (segment (start 156.525 92.475) (end 159 92.475) (width 0.25) (layer "B.Cu") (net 7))
 (segment (start 178.8 80) (end 183.8 85) (width 0.25) (layer "B.Cu") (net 7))
 (segment (start 154 72) (end 196 72) (width 0.25) (layer "F.Cu") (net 3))
 (segment (start 151 75) (end 154 72) (width 0.25) (layer "B.Cu") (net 3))
 (segment (start 173.46 109.5) (end 176 109.5) (width 0.25) (layer "B.Cu") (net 3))
 (segment (start 168.38 109.5) (end 170.92 109.5) (width 0.25) (layer "B.Cu") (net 3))
 (segment (start 157.7 111.15) (end 156 112.85) (width 0.25) (layer "B.Cu") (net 3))
 (segment (start 156 116) (end 158 118) (width 0.25) (layer "B.Cu") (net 3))
 (segment (start 158 118) (end 165 118) (width 0.25) (layer "B.Cu") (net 3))
 (segment (start 156 112.85) (end 156 116) (width 0.25) (layer "B.Cu") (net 3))
 (segment (start 155.55 109) (end 157.7 111.15) (width 0.25) (layer "B.Cu") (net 3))
 (segment (start 153 109) (end 155.55 109) (width 0.25) (layer "B.Cu") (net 3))
 (segment (start 165 118) (end 166 117) (width 0.25) (layer "B.Cu") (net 3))
 (segment (start 166 111.88) (end 168.38 109.5) (width 0.25) (layer "B.Cu") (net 3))
 (segment (start 151 107) (end 151 75) (width 0.25) (layer "B.Cu") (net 3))
 (segment (start 170.92 109.5) (end 173.46 109.5) (width 0.25) (layer "B.Cu") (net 3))
 (segment (start 166 117) (end 166 111.88) (width 0.25) (layer "B.Cu") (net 3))
 (segment (start 153 109) (end 151 107) (width 0.25) (layer "B.Cu") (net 3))
 (segment (start 194 66) (end 191 63) (width 0.25) (layer "B.Cu") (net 35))
 (segment (start 196.2 76.72) (end 196.72 76.72) (width 0.25) (layer "B.Cu") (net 35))
 (segment (start 191 63) (end 188 63) (width 0.25) (layer "B.Cu") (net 35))
 (segment (start 176.495 67) (end 186.25 67) (width 0.25) (layer "B.Cu") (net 35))
 (segment (start 194 79) (end 194 66) (width 0.25) (layer "B.Cu") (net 35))
 (segment (start 188 63) (end 186.25 64.75) (width 0.25) (layer "B.Cu") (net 35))
 (segment (start 186.25 64.75) (end 186.25 67) (width 0.25) (layer "B.Cu") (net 35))
 (segment (start 173.73 64.235) (end 176.495 67) (width 0.25) (layer "B.Cu") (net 35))
 (segment (start 173.99 101.59) (end 171.58 104) (width 0.25) (layer "F.Cu") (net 15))
 (segment (start 171.58 104) (end 169 104) (width 0.25) (layer "F.Cu") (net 15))
 (segment (start 169 104) (end 168.38 104.62) (width 0.25) (layer "F.Cu") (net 15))
 (segment (start 173.99 101.58) (end 173.99 102.01) (width 0.25) (layer "F.Cu") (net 15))
 (segment (start 168.38 104.62) (end 168.38 106.7) (width 0.25) (layer "F.Cu") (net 15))
 (segment (start 174.12 104) (end 173 104) (width 0.25) (layer "F.Cu") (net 16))
 (segment (start 170.92 106.08) (end 170.92 106.7) (width 0.25) (layer "F.Cu") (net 16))
 (segment (start 173 104) (end 170.92 106.08) (width 0.25) (layer "F.Cu") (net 16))
 (segment (start 176.53 101.59) (end 174.12 104) (width 0.25) (layer "F.Cu") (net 16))
 (segment (start 175 104) (end 173.46 105.54) (width 0.25) (layer "F.Cu") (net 17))
 (segment (start 174.1 106.2) (end 174.1 106.96) (width 0.25) (layer "F.Cu") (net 17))
 (segment (start 173.46 105.54) (end 173.46 106.7) (width 0.25) (layer "F.Cu") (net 17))
 (segment (start 176.66 104) (end 175 104) (width 0.25) (layer "F.Cu") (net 17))
 (segment (start 179.07 101.59) (end 176.66 104) (width 0.25) (layer "F.Cu") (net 17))
 (segment (start 181.61 101.59) (end 176.5 106.7) (width 0.25) (layer "F.Cu") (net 18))
 (segment (start 176.5 106.7) (end 176 106.7) (width 0.25) (layer "F.Cu") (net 18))
 (segment (start 155.54 108.46) (end 155.54 111.54) (width 0.25) (layer "F.Cu") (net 4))
 (segment (start 153 111.54) (end 155.54 111.54) (width 0.25) (layer "F.Cu") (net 4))
 (segment (start 159.6 107) (end 157 107) (width 0.25) (layer "F.Cu") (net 4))
 (segment (start 155.54 111.54) (end 159 115) (width 0.25) (layer "F.Cu") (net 4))
 (segment (start 157 107) (end 155.54 108.46) (width 0.25) (layer "F.Cu") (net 4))
 (segment (start 196 69.46) (end 193.54 67) (width 0.25) (layer "F.Cu") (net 34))
 (segment (start 193.54 67) (end 189.75 67) (width 0.25) (layer "F.Cu") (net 34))
 (segment (start 154 69.46) (end 161.04 69.46) (width 0.25) (layer "F.Cu") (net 2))
 (segment (start 161.04 69.46) (end 163.5 67) (width 0.25) (layer "F.Cu") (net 2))
 (segment (start 186.7 80.28) (end 184.5375 78.1175) (width 0.25) (layer "B.Cu") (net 39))
 (segment (start 184.5375 78.1175) (end 184.5375 72) (width 0.25) (layer "B.Cu") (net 39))
 (segment (start 171.19 64.235) (end 171.19 66) (width 0.25) (layer "B.Cu") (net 39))
 (segment (start 183 72) (end 184.5375 72) (width 0.25) (layer "B.Cu") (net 39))
 (segment (start 181 70) (end 183 72) (width 0.25) (layer "B.Cu") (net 39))
 (segment (start 175.19 70) (end 181 70) (width 0.25) (layer "B.Cu") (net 39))
 (segment (start 187.7 80.28) (end 186.7 80.28) (width 0.25) (layer "B.Cu") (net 39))
 (segment (start 171.19 66) (end 175.19 70) (width 0.25) (layer "B.Cu") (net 39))
 (segment (start 168 62) (end 166 64) (width 0.25) (layer "B.Cu") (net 40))
 (segment (start 166 64) (end 166 69) (width 0.25) (layer "B.Cu") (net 40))
 (segment (start 163 72) (end 163 71) (width 0.25) (layer "B.Cu") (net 40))
 (segment (start 176.27 63.235) (end 175.035 62) (width 0.25) (layer "B.Cu") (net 40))
 (segment (start 162.2 75.72) (end 162.2 72.8) (width 0.25) (layer "B.Cu") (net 40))
 (segment (start 166 69) (end 163 72) (width 0.25) (layer "B.Cu") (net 40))
 (segment (start 162.2 72.8) (end 163 72) (width 0.25) (layer "B.Cu") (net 40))
 (segment (start 175.035 62) (end 168 62) (width 0.25) (layer "B.Cu") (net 40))
 (segment (start 178.81 62.81) (end 178.81 63.235) (width 0.25) (layer "B.Cu") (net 1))
 (segment (start 166 61) (end 177 61) (width 0.25) (layer "B.Cu") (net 1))
 (segment (start 155.9 79) (end 155.9 75.1) (width 0.25) (layer "B.Cu") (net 1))
 (segment (start 160 71) (end 160 67) (width 0.25) (layer "B.Cu") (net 1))
 (segment (start 155.9 75.1) (end 160 71) (width 0.25) (layer "B.Cu") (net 1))
 (segment (start 160.1 67.1) (end 160 67) (width 0.25) (layer "B.Cu") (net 1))
 (segment (start 160 67) (end 166 61) (width 0.25) (layer "B.Cu") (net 1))
 (segment (start 177 61) (end 178.81 62.81) (width 0.25) (layer "B.Cu") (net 1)))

